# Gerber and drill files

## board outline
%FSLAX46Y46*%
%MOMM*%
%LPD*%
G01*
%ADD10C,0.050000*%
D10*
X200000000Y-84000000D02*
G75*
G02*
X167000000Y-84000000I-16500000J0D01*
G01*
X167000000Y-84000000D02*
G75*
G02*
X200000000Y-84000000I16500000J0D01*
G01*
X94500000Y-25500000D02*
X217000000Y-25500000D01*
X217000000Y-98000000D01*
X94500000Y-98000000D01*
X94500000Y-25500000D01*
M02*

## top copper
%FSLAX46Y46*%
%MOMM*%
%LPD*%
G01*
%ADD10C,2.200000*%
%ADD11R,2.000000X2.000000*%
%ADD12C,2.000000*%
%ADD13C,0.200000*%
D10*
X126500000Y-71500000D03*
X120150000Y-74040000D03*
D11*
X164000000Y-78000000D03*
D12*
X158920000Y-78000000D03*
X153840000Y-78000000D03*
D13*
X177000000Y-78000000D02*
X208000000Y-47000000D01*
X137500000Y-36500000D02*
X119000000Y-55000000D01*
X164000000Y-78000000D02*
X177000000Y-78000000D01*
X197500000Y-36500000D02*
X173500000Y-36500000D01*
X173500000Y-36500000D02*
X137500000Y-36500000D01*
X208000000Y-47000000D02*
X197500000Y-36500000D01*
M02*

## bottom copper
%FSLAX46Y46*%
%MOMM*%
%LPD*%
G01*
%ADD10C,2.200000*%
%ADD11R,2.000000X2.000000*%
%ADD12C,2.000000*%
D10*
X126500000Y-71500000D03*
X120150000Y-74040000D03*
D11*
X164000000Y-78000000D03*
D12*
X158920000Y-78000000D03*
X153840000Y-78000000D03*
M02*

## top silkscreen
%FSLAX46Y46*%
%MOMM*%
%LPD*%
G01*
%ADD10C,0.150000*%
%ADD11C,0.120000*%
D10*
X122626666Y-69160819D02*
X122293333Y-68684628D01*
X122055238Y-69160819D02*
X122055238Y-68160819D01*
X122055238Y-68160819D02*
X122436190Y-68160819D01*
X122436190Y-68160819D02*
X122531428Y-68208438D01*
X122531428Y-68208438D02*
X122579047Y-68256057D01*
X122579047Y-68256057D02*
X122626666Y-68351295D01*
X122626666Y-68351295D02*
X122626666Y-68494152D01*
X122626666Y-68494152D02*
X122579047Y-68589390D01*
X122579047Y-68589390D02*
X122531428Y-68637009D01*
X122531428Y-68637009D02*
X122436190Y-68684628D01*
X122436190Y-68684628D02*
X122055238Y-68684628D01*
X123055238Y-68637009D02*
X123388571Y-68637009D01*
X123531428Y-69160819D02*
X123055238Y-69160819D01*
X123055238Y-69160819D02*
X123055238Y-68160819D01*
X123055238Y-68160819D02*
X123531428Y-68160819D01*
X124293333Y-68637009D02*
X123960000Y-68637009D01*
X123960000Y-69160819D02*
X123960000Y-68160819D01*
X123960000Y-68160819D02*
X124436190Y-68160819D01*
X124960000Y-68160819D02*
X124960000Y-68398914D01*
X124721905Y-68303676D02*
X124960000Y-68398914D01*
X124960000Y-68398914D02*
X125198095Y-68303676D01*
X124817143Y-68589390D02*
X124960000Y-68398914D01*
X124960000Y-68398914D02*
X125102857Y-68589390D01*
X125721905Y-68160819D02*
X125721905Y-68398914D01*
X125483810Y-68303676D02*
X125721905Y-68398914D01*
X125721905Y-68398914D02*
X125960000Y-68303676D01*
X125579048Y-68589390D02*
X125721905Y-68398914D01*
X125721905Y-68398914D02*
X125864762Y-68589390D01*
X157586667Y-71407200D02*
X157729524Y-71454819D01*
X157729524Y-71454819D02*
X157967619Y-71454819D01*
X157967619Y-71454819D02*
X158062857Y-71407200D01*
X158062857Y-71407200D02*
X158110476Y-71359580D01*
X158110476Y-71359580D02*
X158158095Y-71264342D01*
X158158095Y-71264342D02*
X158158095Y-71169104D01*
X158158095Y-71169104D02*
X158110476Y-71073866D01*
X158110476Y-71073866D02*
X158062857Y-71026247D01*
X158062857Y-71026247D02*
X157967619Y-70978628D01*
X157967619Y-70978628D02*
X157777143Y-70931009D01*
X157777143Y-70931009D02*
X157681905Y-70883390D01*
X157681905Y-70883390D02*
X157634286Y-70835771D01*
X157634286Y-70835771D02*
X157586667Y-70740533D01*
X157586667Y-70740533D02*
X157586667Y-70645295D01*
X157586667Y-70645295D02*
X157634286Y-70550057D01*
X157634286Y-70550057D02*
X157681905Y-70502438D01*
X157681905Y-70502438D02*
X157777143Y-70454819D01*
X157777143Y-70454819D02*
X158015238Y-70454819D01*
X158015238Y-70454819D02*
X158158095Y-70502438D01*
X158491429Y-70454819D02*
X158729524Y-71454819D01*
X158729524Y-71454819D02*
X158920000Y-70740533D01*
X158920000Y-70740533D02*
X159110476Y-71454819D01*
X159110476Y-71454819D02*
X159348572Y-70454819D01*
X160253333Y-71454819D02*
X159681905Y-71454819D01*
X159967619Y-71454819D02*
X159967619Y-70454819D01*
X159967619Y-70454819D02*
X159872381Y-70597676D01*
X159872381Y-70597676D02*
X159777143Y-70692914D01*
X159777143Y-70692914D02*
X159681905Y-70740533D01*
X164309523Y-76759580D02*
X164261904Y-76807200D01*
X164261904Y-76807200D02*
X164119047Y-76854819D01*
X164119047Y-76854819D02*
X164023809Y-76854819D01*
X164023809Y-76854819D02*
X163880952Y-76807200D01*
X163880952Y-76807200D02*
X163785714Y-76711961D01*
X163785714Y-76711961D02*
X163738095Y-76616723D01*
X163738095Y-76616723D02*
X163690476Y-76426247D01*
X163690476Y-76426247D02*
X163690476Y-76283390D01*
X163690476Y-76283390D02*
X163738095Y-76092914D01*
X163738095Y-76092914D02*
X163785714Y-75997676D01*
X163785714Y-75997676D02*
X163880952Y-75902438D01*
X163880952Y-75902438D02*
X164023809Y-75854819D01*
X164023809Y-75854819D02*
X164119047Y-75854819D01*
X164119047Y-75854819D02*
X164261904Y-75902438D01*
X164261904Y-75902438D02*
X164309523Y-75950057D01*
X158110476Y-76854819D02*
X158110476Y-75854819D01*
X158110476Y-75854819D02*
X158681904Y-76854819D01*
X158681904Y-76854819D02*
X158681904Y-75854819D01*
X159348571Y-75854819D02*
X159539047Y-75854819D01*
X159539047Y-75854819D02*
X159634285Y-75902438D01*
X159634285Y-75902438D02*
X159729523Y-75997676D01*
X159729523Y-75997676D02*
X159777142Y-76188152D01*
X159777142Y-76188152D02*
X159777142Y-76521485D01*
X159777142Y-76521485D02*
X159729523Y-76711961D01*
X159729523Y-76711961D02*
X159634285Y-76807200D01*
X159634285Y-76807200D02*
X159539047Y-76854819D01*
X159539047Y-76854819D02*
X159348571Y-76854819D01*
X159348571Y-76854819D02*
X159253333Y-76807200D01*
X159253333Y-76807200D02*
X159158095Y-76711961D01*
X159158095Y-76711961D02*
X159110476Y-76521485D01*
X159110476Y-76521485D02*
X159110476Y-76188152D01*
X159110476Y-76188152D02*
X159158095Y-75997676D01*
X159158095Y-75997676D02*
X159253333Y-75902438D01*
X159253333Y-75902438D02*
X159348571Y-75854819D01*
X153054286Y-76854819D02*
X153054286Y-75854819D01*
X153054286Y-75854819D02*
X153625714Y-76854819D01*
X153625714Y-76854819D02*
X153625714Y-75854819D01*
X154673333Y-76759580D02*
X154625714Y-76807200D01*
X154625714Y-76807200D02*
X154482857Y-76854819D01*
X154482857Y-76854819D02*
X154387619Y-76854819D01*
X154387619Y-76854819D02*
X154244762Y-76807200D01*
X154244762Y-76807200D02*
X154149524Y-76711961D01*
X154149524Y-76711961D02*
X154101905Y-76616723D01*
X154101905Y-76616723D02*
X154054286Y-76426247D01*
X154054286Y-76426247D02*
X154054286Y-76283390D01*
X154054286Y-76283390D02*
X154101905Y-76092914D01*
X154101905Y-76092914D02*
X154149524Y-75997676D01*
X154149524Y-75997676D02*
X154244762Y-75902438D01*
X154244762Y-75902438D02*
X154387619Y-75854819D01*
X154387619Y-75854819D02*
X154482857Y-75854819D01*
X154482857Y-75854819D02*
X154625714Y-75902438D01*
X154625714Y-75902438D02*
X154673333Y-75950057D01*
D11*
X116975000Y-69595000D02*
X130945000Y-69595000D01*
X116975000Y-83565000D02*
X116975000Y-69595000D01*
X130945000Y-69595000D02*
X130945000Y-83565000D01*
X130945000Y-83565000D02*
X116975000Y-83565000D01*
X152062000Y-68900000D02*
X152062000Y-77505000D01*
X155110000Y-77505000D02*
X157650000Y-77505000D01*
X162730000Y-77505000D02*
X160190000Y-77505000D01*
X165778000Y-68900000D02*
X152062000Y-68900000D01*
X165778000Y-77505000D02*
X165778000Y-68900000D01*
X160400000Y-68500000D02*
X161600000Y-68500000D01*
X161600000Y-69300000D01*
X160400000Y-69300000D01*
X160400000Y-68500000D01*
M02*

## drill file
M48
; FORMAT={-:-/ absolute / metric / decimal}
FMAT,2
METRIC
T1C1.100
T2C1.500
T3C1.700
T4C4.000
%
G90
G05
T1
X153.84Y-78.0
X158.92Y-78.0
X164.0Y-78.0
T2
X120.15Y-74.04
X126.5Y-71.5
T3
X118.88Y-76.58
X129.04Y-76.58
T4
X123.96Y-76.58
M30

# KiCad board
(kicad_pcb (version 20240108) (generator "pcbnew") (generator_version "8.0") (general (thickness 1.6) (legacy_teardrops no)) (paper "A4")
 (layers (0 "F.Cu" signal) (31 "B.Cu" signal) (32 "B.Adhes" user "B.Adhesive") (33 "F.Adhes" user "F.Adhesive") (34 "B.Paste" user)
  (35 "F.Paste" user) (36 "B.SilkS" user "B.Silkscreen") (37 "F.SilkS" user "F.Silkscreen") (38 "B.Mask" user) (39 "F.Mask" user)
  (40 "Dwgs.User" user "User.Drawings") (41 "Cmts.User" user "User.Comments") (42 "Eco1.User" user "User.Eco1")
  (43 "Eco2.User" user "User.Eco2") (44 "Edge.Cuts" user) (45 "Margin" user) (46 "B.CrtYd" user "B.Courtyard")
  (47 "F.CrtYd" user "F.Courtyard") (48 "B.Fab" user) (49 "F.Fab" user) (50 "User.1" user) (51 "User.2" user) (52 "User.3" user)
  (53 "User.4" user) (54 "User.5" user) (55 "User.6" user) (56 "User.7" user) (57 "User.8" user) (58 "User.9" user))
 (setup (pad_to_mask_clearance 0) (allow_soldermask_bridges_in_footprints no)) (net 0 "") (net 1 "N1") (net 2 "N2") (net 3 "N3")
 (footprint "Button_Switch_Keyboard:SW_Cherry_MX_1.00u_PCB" (layer "F.Cu") (at 126.5 71.5)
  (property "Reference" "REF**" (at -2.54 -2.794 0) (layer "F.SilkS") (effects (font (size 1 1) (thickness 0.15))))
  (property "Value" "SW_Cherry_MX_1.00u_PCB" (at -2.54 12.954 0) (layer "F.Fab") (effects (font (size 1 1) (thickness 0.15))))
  (fp_line (start -9.525 -1.905) (end 4.445 -1.905) (stroke (width 0.12) (type solid)) (layer "F.SilkS"))
  (fp_line (start -9.525 12.065) (end -9.525 -1.905) (stroke (width 0.12) (type solid)) (layer "F.SilkS"))
  (fp_line (start 4.445 -1.905) (end 4.445 12.065) (stroke (width 0.12) (type solid)) (layer "F.SilkS"))
  (fp_line (start 4.445 12.065) (end -9.525 12.065) (stroke (width 0.12) (type solid)) (layer "F.SilkS"))
  (pad "" np_thru_hole circle (at -7.62 5.08) (size 1.7 1.7) (drill 1.7) (layers "*.Cu" "*.Mask"))
  (pad "" np_thru_hole circle (at -2.54 5.08) (size 4 4) (drill 4) (layers "*.Cu" "*.Mask"))
  (pad "" np_thru_hole circle (at 2.54 5.08) (size 1.7 1.7) (drill 1.7) (layers "*.Cu" "*.Mask"))
  (pad "1" thru_hole circle (at 0 0) (size 2.2 2.2) (drill 1.5) (layers "*.Cu" "*.Mask") (remove_unused_layers no))
  (pad "2" thru_hole circle (at -6.35 2.54) (size 2.2 2.2) (drill 1.5) (layers "*.Cu" "*.Mask") (remove_unused_layers no)))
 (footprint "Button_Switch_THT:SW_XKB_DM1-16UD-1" (layer "F.Cu") (at 164 78)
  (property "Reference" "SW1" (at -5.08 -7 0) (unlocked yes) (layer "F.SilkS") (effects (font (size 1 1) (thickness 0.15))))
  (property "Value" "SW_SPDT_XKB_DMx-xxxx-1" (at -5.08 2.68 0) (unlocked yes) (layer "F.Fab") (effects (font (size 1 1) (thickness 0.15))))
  (fp_line (start -11.938 -9.1) (end -11.938 -0.495) (stroke (width 0.12) (type solid)) (layer "F.SilkS"))
  (fp_line (start -8.89 -0.495) (end -6.35 -0.495) (stroke (width 0.12) (type solid)) (layer "F.SilkS"))
  (fp_line (start -1.27 -0.495) (end -3.81 -0.495) (stroke (width 0.12) (type solid)) (layer "F.SilkS"))
  (fp_line (start 1.778 -9.1) (end -11.938 -9.1) (stroke (width 0.12) (type solid)) (layer "F.SilkS"))
  (fp_line (start 1.778 -0.495) (end 1.778 -9.1) (stroke (width 0.12) (type solid)) (layer "F.SilkS"))
  (fp_rect (start -3.6 -9.5) (end -2.4 -8.7) (stroke (width 0.12) (type solid)) (fill none) (layer "F.SilkS"))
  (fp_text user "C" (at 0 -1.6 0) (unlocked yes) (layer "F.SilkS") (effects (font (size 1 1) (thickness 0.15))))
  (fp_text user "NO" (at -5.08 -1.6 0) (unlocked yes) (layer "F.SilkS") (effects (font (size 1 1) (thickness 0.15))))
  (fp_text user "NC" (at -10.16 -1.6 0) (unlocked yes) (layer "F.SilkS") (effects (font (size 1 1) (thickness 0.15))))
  (pad "1" thru_hole rect (at 0 0) (size 2 2) (drill 1.1) (layers "*.Cu" "*.Mask") (remove_unused_layers no) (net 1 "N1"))
  (pad "2" thru_hole circle (at -5.08 0) (size 2 2) (drill 1.1) (layers "*.Cu" "*.Mask") (remove_unused_layers no) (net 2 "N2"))
  (pad "3" thru_hole circle (at -10.16 0) (size 2 2) (drill 1.1) (layers "*.Cu" "*.Mask") (remove_unused_layers no) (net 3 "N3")))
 (gr_circle (center 183.5 84) (end 200 84) (stroke (width 0.05) (type default)) (fill none) (layer "Edge.Cuts"))
 (gr_rect (start 94.5 25.5) (end 217 98) (stroke (width 0.05) (type default)) (fill none) (layer "Edge.Cuts"))
 (segment (start 177 78) (end 208 47) (width 0.2) (layer "F.Cu") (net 1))
 (segment (start 137.5 36.5) (end 119 55) (width 0.2) (layer "F.Cu") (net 1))
 (segment (start 164 78) (end 177 78) (width 0.2) (layer "F.Cu") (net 1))
 (segment (start 197.5 36.5) (end 173.5 36.5) (width 0.2) (layer "F.Cu") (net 1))
 (segment (start 173.5 36.5) (end 137.5 36.5) (width 0.2) (layer "F.Cu") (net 1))
 (segment (start 208 47) (end 197.5 36.5) (width 0.2) (layer "F.Cu") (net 1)))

